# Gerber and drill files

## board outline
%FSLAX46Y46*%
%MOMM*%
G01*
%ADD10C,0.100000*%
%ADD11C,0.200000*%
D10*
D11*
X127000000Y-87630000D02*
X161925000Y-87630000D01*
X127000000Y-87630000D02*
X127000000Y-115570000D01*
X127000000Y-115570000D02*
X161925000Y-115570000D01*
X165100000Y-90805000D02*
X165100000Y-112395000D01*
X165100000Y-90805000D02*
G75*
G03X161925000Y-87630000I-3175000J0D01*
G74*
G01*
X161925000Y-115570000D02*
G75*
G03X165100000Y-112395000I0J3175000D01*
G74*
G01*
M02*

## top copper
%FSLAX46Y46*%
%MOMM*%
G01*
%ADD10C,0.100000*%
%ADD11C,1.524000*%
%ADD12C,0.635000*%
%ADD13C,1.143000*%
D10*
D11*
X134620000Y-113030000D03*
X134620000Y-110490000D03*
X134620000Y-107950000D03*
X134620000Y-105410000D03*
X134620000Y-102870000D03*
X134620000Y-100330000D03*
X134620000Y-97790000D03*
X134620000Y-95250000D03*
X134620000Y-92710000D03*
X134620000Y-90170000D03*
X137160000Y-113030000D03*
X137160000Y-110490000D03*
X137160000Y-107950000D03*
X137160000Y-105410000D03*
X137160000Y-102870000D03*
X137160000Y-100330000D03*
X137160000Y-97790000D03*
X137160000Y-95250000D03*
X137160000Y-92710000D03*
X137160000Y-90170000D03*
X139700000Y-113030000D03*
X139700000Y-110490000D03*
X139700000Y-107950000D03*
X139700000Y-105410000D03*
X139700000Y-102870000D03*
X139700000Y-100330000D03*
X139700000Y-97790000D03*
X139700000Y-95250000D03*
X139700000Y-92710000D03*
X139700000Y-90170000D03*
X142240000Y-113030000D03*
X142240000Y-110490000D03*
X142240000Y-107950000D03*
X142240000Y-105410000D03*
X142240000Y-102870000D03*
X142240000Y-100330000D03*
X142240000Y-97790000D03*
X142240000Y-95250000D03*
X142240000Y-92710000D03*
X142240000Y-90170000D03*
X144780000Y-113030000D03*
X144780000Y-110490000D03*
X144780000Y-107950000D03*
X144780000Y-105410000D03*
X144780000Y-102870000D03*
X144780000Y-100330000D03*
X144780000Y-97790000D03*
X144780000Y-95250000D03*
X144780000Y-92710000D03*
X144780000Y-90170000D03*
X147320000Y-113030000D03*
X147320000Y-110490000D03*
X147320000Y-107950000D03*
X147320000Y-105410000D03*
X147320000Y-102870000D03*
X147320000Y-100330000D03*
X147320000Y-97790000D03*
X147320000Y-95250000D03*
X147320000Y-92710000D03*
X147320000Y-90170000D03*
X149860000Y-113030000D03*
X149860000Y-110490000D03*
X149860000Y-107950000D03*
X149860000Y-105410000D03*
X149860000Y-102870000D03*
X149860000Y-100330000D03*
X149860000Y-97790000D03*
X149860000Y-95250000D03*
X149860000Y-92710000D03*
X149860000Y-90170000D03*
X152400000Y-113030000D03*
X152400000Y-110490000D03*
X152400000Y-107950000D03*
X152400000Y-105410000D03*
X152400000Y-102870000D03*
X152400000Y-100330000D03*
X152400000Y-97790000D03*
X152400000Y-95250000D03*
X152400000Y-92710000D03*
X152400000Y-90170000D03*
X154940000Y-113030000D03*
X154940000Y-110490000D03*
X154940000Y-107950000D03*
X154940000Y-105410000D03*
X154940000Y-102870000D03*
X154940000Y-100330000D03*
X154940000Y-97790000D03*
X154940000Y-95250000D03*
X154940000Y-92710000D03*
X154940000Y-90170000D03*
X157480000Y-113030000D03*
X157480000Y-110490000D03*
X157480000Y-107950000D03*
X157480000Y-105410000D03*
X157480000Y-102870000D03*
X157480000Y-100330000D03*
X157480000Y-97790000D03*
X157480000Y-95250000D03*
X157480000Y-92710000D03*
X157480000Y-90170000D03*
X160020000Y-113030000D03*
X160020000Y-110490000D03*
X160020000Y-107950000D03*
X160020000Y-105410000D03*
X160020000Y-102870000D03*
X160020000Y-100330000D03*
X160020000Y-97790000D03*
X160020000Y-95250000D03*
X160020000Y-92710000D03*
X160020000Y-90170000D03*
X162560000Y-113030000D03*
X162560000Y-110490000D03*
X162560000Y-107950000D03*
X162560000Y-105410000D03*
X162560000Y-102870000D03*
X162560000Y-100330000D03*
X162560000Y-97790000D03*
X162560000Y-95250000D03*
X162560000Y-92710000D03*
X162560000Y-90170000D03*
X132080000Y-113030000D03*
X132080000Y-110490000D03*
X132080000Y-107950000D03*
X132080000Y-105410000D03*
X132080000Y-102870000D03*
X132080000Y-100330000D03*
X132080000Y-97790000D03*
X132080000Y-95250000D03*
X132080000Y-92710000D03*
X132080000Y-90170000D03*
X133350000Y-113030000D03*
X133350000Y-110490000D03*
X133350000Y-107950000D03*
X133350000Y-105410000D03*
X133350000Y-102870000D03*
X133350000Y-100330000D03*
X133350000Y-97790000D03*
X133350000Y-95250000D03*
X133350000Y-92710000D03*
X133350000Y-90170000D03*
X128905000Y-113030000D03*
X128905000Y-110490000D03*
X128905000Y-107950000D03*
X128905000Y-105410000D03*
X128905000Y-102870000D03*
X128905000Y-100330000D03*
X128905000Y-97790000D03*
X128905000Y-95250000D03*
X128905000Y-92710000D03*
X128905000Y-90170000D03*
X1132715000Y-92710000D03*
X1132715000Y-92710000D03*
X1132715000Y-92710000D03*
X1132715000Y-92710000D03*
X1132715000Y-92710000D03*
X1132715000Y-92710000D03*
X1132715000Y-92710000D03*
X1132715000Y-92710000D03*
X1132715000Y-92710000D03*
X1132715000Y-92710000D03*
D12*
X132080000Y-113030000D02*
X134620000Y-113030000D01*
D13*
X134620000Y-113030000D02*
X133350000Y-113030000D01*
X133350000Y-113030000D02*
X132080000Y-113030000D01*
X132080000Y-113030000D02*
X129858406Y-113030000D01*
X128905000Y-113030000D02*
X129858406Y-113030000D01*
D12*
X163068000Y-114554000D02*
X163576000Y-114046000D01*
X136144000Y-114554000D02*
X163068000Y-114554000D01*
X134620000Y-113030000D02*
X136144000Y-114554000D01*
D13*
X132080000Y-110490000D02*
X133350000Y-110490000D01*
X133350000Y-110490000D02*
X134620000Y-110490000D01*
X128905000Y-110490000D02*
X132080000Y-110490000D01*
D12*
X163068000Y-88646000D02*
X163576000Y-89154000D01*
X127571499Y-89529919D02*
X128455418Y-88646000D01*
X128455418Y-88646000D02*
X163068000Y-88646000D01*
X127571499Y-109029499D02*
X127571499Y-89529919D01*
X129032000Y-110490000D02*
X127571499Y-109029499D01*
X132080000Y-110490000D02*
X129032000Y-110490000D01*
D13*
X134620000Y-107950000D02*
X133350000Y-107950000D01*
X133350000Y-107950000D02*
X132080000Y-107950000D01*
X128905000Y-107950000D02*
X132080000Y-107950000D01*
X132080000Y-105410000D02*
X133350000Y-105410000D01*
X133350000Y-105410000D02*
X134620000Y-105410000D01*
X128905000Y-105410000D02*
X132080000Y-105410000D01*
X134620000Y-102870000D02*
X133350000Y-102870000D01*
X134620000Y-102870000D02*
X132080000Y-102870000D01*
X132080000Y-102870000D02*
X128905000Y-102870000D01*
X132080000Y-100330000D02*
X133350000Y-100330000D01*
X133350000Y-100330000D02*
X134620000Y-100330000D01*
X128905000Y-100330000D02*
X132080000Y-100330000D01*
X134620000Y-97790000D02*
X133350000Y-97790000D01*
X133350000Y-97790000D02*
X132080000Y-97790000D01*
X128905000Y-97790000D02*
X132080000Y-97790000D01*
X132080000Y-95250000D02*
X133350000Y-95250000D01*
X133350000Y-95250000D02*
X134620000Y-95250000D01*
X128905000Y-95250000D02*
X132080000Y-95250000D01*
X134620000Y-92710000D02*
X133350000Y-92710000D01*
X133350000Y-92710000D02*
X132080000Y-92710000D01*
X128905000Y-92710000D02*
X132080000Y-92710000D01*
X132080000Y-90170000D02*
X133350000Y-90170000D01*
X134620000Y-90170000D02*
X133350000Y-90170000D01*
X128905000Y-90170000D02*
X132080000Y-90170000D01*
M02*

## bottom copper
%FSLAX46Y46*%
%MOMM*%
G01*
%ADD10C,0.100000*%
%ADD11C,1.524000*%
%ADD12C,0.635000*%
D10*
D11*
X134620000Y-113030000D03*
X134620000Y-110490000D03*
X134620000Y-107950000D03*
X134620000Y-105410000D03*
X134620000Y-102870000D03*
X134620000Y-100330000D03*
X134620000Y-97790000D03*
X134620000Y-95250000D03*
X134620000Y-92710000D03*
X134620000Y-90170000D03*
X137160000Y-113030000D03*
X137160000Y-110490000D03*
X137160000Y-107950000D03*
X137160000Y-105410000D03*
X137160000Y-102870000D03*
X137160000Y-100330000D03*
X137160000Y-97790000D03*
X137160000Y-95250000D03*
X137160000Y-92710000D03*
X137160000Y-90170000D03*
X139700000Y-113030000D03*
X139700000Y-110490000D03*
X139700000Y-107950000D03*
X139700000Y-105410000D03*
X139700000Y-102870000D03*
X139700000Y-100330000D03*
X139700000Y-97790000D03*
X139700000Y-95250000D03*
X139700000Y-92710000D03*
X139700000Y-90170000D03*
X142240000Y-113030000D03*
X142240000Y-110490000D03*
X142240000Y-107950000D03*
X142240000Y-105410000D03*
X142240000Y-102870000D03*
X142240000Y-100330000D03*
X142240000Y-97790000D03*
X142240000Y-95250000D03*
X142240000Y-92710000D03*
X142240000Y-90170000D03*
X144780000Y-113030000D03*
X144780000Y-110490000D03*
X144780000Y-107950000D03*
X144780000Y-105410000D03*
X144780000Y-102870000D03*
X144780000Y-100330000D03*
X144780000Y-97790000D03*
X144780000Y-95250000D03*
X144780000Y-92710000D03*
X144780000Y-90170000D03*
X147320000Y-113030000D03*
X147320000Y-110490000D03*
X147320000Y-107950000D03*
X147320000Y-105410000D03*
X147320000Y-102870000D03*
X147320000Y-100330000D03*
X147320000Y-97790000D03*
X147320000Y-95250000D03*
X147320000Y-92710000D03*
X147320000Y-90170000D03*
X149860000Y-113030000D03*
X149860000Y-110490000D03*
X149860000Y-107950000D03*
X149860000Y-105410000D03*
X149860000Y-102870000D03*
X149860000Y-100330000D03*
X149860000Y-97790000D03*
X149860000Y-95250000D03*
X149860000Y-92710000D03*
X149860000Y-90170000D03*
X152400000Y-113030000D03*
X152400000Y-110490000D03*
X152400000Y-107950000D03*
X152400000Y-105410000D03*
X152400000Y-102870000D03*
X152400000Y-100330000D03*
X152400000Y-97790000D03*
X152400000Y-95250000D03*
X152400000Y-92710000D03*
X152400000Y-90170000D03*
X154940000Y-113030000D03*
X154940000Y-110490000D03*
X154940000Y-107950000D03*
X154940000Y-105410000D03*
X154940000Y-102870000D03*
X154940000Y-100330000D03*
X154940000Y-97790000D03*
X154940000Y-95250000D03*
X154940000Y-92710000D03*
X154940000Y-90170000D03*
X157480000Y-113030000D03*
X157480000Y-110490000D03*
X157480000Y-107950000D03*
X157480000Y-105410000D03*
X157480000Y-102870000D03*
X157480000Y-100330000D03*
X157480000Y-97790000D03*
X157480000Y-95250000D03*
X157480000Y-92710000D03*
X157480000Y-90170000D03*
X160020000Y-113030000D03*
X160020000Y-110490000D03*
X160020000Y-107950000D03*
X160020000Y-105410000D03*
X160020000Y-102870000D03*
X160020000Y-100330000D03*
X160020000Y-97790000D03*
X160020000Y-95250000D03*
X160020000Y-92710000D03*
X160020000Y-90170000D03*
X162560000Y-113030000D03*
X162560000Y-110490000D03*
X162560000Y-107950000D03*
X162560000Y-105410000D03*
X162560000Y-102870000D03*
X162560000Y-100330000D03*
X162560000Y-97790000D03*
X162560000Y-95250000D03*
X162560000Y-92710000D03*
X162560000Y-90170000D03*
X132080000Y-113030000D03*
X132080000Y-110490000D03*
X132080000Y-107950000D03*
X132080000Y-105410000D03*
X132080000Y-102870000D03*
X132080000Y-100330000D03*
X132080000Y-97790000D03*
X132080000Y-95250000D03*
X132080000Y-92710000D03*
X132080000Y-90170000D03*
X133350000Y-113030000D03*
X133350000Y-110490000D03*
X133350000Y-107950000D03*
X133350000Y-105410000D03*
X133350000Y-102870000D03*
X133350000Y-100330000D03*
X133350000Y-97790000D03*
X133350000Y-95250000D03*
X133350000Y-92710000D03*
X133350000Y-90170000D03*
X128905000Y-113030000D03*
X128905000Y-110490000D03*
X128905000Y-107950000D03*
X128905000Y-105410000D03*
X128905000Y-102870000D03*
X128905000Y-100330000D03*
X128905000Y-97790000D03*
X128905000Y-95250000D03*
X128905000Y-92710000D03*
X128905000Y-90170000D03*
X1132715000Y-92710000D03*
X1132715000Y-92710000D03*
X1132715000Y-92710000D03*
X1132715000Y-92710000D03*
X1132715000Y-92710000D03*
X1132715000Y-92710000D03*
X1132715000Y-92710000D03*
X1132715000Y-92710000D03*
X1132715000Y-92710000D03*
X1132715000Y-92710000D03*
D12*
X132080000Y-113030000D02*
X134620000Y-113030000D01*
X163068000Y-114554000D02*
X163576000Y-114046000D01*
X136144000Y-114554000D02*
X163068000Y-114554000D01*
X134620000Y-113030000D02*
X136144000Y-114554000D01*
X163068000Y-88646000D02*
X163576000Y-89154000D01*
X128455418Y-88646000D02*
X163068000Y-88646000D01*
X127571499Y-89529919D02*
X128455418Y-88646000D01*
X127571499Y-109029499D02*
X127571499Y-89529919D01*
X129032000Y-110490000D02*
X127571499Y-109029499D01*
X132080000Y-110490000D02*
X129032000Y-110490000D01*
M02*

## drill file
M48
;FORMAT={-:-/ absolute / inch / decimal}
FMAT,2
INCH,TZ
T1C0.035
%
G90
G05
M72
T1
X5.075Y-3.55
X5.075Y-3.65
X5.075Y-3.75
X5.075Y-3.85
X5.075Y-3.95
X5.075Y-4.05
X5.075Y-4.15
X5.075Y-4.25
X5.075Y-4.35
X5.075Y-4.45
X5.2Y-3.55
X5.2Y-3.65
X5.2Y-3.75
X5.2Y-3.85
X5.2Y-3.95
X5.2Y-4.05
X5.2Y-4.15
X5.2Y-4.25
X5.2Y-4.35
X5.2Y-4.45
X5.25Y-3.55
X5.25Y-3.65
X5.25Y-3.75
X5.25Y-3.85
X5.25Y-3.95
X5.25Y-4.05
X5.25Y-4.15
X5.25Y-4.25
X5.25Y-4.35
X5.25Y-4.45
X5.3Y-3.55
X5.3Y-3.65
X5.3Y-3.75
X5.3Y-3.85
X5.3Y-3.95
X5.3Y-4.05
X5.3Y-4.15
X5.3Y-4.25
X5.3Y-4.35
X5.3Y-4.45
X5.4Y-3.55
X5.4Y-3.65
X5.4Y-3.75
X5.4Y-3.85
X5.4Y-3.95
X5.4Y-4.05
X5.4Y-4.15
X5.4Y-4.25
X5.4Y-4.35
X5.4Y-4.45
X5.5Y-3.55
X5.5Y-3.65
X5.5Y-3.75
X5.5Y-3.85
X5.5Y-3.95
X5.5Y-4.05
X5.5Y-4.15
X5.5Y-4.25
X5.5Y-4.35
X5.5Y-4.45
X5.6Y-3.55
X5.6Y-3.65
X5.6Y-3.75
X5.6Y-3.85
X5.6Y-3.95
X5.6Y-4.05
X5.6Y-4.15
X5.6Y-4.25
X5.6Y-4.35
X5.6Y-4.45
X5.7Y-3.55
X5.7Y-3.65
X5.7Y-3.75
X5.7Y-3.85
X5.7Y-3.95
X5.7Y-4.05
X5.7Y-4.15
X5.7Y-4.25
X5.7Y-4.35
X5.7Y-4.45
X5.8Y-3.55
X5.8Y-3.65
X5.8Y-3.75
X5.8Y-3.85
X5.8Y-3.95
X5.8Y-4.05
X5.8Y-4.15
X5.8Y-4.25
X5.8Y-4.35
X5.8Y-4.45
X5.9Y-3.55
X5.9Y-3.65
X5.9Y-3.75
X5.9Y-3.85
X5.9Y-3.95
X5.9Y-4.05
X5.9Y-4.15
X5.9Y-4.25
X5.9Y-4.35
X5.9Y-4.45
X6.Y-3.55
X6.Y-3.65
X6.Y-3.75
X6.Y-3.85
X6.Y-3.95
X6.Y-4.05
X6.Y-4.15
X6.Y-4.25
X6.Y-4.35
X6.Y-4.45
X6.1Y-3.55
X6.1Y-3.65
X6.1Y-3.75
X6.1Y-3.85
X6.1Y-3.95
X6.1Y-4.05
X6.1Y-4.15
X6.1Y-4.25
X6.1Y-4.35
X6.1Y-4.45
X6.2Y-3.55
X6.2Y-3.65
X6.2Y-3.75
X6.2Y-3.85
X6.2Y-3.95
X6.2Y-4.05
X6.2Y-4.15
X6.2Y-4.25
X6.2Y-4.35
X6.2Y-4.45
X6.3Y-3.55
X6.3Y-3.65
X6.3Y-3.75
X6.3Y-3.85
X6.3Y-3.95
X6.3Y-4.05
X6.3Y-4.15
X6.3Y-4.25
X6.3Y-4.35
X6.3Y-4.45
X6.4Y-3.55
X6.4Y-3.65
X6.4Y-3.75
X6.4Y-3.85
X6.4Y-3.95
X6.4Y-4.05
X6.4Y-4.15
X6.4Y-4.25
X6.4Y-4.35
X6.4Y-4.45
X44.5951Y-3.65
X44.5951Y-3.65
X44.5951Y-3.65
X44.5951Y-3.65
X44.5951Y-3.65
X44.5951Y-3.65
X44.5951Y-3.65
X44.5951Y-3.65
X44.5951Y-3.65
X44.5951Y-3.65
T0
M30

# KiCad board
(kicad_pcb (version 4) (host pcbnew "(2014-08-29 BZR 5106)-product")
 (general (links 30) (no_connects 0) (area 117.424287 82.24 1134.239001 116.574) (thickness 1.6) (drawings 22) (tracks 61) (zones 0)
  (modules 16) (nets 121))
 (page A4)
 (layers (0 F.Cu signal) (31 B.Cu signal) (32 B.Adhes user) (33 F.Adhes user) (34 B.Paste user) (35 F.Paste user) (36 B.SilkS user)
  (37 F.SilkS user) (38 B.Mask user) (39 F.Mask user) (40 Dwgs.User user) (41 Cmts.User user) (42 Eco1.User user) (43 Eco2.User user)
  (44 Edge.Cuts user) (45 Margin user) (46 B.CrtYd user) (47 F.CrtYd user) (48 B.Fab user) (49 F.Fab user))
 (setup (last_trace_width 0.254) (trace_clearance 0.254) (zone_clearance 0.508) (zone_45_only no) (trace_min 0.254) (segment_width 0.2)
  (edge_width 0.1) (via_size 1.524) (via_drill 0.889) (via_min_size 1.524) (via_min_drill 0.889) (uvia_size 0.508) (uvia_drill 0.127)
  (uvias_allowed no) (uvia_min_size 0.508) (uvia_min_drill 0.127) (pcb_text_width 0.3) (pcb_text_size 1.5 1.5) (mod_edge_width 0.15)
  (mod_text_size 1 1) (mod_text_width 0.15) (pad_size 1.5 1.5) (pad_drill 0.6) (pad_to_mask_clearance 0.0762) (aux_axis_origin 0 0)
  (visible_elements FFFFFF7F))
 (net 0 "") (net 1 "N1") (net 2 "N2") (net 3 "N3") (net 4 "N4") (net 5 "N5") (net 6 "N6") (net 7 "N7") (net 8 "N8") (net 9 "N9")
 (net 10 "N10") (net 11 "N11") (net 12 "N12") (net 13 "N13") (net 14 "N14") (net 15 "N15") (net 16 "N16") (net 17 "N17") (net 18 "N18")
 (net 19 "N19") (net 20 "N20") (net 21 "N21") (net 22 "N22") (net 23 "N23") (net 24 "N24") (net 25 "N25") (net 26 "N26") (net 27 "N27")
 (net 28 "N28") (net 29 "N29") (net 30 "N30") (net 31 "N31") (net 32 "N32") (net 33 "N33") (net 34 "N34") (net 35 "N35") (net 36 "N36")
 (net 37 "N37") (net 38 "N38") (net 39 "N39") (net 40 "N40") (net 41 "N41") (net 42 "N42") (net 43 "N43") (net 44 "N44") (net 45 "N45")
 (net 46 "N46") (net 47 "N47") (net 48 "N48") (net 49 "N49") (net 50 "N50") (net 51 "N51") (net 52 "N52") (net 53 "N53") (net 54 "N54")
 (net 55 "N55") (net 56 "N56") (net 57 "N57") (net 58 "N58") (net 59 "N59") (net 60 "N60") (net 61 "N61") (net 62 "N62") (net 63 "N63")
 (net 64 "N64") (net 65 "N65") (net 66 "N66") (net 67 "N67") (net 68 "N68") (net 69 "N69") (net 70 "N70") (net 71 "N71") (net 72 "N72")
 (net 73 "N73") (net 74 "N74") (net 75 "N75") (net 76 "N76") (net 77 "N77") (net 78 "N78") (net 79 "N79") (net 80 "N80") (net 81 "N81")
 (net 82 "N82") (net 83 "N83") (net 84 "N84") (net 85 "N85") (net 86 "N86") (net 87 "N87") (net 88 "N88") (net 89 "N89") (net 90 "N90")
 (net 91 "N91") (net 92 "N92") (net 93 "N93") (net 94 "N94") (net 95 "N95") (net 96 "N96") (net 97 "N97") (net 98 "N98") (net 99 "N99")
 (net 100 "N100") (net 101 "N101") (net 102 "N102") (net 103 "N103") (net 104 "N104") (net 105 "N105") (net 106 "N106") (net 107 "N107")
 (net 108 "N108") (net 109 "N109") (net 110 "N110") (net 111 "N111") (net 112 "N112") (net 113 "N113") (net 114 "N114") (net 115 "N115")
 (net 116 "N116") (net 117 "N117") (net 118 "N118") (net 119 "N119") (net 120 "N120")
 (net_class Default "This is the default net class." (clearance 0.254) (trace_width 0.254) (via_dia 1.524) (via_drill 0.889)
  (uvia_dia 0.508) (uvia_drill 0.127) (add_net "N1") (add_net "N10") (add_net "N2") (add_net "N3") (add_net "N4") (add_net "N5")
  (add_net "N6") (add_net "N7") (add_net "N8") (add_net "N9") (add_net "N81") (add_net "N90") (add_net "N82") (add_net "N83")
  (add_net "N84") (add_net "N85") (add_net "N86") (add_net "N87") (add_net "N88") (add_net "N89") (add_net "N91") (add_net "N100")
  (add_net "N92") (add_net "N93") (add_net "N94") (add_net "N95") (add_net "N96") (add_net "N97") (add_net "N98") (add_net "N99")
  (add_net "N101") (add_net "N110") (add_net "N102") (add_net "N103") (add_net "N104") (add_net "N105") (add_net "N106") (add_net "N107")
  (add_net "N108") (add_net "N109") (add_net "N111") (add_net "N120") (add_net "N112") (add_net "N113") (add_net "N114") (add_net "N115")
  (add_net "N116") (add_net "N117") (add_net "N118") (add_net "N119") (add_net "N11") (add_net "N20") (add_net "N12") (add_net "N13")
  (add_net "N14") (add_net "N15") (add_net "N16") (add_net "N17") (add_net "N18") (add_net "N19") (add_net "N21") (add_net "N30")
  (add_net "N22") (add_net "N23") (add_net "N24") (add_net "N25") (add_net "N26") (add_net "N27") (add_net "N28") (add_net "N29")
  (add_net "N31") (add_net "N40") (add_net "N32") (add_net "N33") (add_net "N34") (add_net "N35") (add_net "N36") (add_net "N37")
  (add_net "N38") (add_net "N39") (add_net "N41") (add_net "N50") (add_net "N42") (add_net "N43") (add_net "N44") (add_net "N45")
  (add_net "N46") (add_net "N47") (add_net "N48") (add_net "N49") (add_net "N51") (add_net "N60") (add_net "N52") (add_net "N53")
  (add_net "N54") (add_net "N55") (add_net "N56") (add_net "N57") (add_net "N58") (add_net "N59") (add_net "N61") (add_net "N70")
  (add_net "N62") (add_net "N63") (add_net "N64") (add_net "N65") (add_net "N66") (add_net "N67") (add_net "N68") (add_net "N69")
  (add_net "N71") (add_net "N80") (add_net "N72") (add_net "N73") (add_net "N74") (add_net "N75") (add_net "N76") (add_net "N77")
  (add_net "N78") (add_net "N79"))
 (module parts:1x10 (layer F.Cu) (at 134.62 101.6 90)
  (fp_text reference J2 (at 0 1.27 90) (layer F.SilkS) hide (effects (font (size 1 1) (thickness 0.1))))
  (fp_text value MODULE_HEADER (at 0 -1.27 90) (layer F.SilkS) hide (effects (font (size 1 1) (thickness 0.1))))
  (pad 1 thru_hole circle (at -11.43 0 90) (size 1.524 1.524) (drill 0.889) (layers *.Cu *.Mask F.SilkS) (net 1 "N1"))
  (pad 2 thru_hole circle (at -8.89 0 90) (size 1.524 1.524) (drill 0.889) (layers *.Cu *.Mask F.SilkS) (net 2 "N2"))
  (pad 3 thru_hole circle (at -6.35 0 90) (size 1.524 1.524) (drill 0.889) (layers *.Cu *.Mask F.SilkS) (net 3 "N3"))
  (pad 4 thru_hole circle (at -3.81 0 90) (size 1.524 1.524) (drill 0.889) (layers *.Cu *.Mask F.SilkS) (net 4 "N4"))
  (pad 5 thru_hole circle (at -1.27 0 90) (size 1.524 1.524) (drill 0.889) (layers *.Cu *.Mask F.SilkS) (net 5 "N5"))
  (pad 6 thru_hole circle (at 1.27 0 90) (size 1.524 1.524) (drill 0.889) (layers *.Cu *.Mask F.SilkS) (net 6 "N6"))
  (pad 7 thru_hole circle (at 3.81 0 90) (size 1.524 1.524) (drill 0.889) (layers *.Cu *.Mask F.SilkS) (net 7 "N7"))
  (pad 8 thru_hole circle (at 6.35 0 90) (size 1.524 1.524) (drill 0.889) (layers *.Cu *.Mask F.SilkS) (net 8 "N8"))
  (pad 9 thru_hole circle (at 8.89 0 90) (size 1.524 1.524) (drill 0.889) (layers *.Cu *.Mask F.SilkS) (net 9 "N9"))
  (pad 10 thru_hole circle (at 11.43 0 90) (size 1.524 1.524) (drill 0.889) (layers *.Cu *.Mask F.SilkS) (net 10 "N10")))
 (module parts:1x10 (layer F.Cu) (at 137.16 101.6 90)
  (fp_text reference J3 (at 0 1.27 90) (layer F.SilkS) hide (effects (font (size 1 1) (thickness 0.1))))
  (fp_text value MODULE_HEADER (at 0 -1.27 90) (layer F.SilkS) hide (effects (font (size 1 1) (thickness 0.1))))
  (pad 1 thru_hole circle (at -11.43 0 90) (size 1.524 1.524) (drill 0.889) (layers *.Cu *.Mask F.SilkS) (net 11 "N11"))
  (pad 2 thru_hole circle (at -8.89 0 90) (size 1.524 1.524) (drill 0.889) (layers *.Cu *.Mask F.SilkS) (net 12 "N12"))
  (pad 3 thru_hole circle (at -6.35 0 90) (size 1.524 1.524) (drill 0.889) (layers *.Cu *.Mask F.SilkS) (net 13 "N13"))
  (pad 4 thru_hole circle (at -3.81 0 90) (size 1.524 1.524) (drill 0.889) (layers *.Cu *.Mask F.SilkS) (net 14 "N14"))
  (pad 5 thru_hole circle (at -1.27 0 90) (size 1.524 1.524) (drill 0.889) (layers *.Cu *.Mask F.SilkS) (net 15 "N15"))
  (pad 6 thru_hole circle (at 1.27 0 90) (size 1.524 1.524) (drill 0.889) (layers *.Cu *.Mask F.SilkS) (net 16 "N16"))
  (pad 7 thru_hole circle (at 3.81 0 90) (size 1.524 1.524) (drill 0.889) (layers *.Cu *.Mask F.SilkS) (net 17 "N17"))
  (pad 8 thru_hole circle (at 6.35 0 90) (size 1.524 1.524) (drill 0.889) (layers *.Cu *.Mask F.SilkS) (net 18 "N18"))
  (pad 9 thru_hole circle (at 8.89 0 90) (size 1.524 1.524) (drill 0.889) (layers *.Cu *.Mask F.SilkS) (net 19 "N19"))
  (pad 10 thru_hole circle (at 11.43 0 90) (size 1.524 1.524) (drill 0.889) (layers *.Cu *.Mask F.SilkS) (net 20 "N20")))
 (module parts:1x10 (layer F.Cu) (at 139.7 101.6 90)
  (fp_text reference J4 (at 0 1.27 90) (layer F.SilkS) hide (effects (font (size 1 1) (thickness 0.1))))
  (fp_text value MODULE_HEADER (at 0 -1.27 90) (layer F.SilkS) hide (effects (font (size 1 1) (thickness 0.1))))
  (pad 1 thru_hole circle (at -11.43 0 90) (size 1.524 1.524) (drill 0.889) (layers *.Cu *.Mask F.SilkS) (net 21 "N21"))
  (pad 2 thru_hole circle (at -8.89 0 90) (size 1.524 1.524) (drill 0.889) (layers *.Cu *.Mask F.SilkS) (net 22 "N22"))
  (pad 3 thru_hole circle (at -6.35 0 90) (size 1.524 1.524) (drill 0.889) (layers *.Cu *.Mask F.SilkS) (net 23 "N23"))
  (pad 4 thru_hole circle (at -3.81 0 90) (size 1.524 1.524) (drill 0.889) (layers *.Cu *.Mask F.SilkS) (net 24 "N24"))
  (pad 5 thru_hole circle (at -1.27 0 90) (size 1.524 1.524) (drill 0.889) (layers *.Cu *.Mask F.SilkS) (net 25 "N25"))
  (pad 6 thru_hole circle (at 1.27 0 90) (size 1.524 1.524) (drill 0.889) (layers *.Cu *.Mask F.SilkS) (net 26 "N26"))
  (pad 7 thru_hole circle (at 3.81 0 90) (size 1.524 1.524) (drill 0.889) (layers *.Cu *.Mask F.SilkS) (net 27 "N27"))
  (pad 8 thru_hole circle (at 6.35 0 90) (size 1.524 1.524) (drill 0.889) (layers *.Cu *.Mask F.SilkS) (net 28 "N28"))
  (pad 9 thru_hole circle (at 8.89 0 90) (size 1.524 1.524) (drill 0.889) (layers *.Cu *.Mask F.SilkS) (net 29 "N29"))
  (pad 10 thru_hole circle (at 11.43 0 90) (size 1.524 1.524) (drill 0.889) (layers *.Cu *.Mask F.SilkS) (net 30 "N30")))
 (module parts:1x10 (layer F.Cu) (at 142.24 101.6 90)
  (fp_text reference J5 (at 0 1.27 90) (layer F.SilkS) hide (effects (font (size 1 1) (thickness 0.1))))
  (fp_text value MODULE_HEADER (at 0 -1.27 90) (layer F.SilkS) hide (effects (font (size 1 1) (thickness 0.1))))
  (pad 1 thru_hole circle (at -11.43 0 90) (size 1.524 1.524) (drill 0.889) (layers *.Cu *.Mask F.SilkS) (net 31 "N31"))
  (pad 2 thru_hole circle (at -8.89 0 90) (size 1.524 1.524) (drill 0.889) (layers *.Cu *.Mask F.SilkS) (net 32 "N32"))
  (pad 3 thru_hole circle (at -6.35 0 90) (size 1.524 1.524) (drill 0.889) (layers *.Cu *.Mask F.SilkS) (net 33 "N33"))
  (pad 4 thru_hole circle (at -3.81 0 90) (size 1.524 1.524) (drill 0.889) (layers *.Cu *.Mask F.SilkS) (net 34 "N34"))
  (pad 5 thru_hole circle (at -1.27 0 90) (size 1.524 1.524) (drill 0.889) (layers *.Cu *.Mask F.SilkS) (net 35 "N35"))
  (pad 6 thru_hole circle (at 1.27 0 90) (size 1.524 1.524) (drill 0.889) (layers *.Cu *.Mask F.SilkS) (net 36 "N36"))
  (pad 7 thru_hole circle (at 3.81 0 90) (size 1.524 1.524) (drill 0.889) (layers *.Cu *.Mask F.SilkS) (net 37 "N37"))
  (pad 8 thru_hole circle (at 6.35 0 90) (size 1.524 1.524) (drill 0.889) (layers *.Cu *.Mask F.SilkS) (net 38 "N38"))
  (pad 9 thru_hole circle (at 8.89 0 90) (size 1.524 1.524) (drill 0.889) (layers *.Cu *.Mask F.SilkS) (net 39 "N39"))
  (pad 10 thru_hole circle (at 11.43 0 90) (size 1.524 1.524) (drill 0.889) (layers *.Cu *.Mask F.SilkS) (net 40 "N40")))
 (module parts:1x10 (layer F.Cu) (at 144.78 101.6 90)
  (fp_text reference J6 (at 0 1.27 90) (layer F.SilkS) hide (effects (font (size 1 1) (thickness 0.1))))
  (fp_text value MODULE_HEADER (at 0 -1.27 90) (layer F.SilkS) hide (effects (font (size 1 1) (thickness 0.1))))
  (pad 1 thru_hole circle (at -11.43 0 90) (size 1.524 1.524) (drill 0.889) (layers *.Cu *.Mask F.SilkS) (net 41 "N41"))
  (pad 2 thru_hole circle (at -8.89 0 90) (size 1.524 1.524) (drill 0.889) (layers *.Cu *.Mask F.SilkS) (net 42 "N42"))
  (pad 3 thru_hole circle (at -6.35 0 90) (size 1.524 1.524) (drill 0.889) (layers *.Cu *.Mask F.SilkS) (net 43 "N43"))
  (pad 4 thru_hole circle (at -3.81 0 90) (size 1.524 1.524) (drill 0.889) (layers *.Cu *.Mask F.SilkS) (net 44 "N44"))
  (pad 5 thru_hole circle (at -1.27 0 90) (size 1.524 1.524) (drill 0.889) (layers *.Cu *.Mask F.SilkS) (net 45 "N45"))
  (pad 6 thru_hole circle (at 1.27 0 90) (size 1.524 1.524) (drill 0.889) (layers *.Cu *.Mask F.SilkS) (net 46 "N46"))
  (pad 7 thru_hole circle (at 3.81 0 90) (size 1.524 1.524) (drill 0.889) (layers *.Cu *.Mask F.SilkS) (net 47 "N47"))
  (pad 8 thru_hole circle (at 6.35 0 90) (size 1.524 1.524) (drill 0.889) (layers *.Cu *.Mask F.SilkS) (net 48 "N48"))
  (pad 9 thru_hole circle (at 8.89 0 90) (size 1.524 1.524) (drill 0.889) (layers *.Cu *.Mask F.SilkS) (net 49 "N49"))
  (pad 10 thru_hole circle (at 11.43 0 90) (size 1.524 1.524) (drill 0.889) (layers *.Cu *.Mask F.SilkS) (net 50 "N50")))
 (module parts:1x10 (layer F.Cu) (at 147.32 101.6 90)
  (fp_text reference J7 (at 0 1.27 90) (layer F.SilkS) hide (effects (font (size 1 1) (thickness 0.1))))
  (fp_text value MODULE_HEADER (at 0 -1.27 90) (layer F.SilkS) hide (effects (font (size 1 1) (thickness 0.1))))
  (pad 1 thru_hole circle (at -11.43 0 90) (size 1.524 1.524) (drill 0.889) (layers *.Cu *.Mask F.SilkS) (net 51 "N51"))
  (pad 2 thru_hole circle (at -8.89 0 90) (size 1.524 1.524) (drill 0.889) (layers *.Cu *.Mask F.SilkS) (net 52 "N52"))
  (pad 3 thru_hole circle (at -6.35 0 90) (size 1.524 1.524) (drill 0.889) (layers *.Cu *.Mask F.SilkS) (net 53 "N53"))
  (pad 4 thru_hole circle (at -3.81 0 90) (size 1.524 1.524) (drill 0.889) (layers *.Cu *.Mask F.SilkS) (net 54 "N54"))
  (pad 5 thru_hole circle (at -1.27 0 90) (size 1.524 1.524) (drill 0.889) (layers *.Cu *.Mask F.SilkS) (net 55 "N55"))
  (pad 6 thru_hole circle (at 1.27 0 90) (size 1.524 1.524) (drill 0.889) (layers *.Cu *.Mask F.SilkS) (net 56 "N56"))
  (pad 7 thru_hole circle (at 3.81 0 90) (size 1.524 1.524) (drill 0.889) (layers *.Cu *.Mask F.SilkS) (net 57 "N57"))
  (pad 8 thru_hole circle (at 6.35 0 90) (size 1.524 1.524) (drill 0.889) (layers *.Cu *.Mask F.SilkS) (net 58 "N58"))
  (pad 9 thru_hole circle (at 8.89 0 90) (size 1.524 1.524) (drill 0.889) (layers *.Cu *.Mask F.SilkS) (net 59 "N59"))
  (pad 10 thru_hole circle (at 11.43 0 90) (size 1.524 1.524) (drill 0.889) (layers *.Cu *.Mask F.SilkS) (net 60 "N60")))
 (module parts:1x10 (layer F.Cu) (at 149.86 101.6 90)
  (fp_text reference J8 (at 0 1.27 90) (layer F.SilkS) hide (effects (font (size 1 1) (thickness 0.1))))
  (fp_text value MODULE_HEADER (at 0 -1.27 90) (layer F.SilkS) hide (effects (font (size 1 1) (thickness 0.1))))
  (pad 1 thru_hole circle (at -11.43 0 90) (size 1.524 1.524) (drill 0.889) (layers *.Cu *.Mask F.SilkS) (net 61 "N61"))
  (pad 2 thru_hole circle (at -8.89 0 90) (size 1.524 1.524) (drill 0.889) (layers *.Cu *.Mask F.SilkS) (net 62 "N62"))
  (pad 3 thru_hole circle (at -6.35 0 90) (size 1.524 1.524) (drill 0.889) (layers *.Cu *.Mask F.SilkS) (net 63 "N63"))
  (pad 4 thru_hole circle (at -3.81 0 90) (size 1.524 1.524) (drill 0.889) (layers *.Cu *.Mask F.SilkS) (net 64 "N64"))
  (pad 5 thru_hole circle (at -1.27 0 90) (size 1.524 1.524) (drill 0.889) (layers *.Cu *.Mask F.SilkS) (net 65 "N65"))
  (pad 6 thru_hole circle (at 1.27 0 90) (size 1.524 1.524) (drill 0.889) (layers *.Cu *.Mask F.SilkS) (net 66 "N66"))
  (pad 7 thru_hole circle (at 3.81 0 90) (size 1.524 1.524) (drill 0.889) (layers *.Cu *.Mask F.SilkS) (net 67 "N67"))
  (pad 8 thru_hole circle (at 6.35 0 90) (size 1.524 1.524) (drill 0.889) (layers *.Cu *.Mask F.SilkS) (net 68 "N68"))
  (pad 9 thru_hole circle (at 8.89 0 90) (size 1.524 1.524) (drill 0.889) (layers *.Cu *.Mask F.SilkS) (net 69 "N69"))
  (pad 10 thru_hole circle (at 11.43 0 90) (size 1.524 1.524) (drill 0.889) (layers *.Cu *.Mask F.SilkS) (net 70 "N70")))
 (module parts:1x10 (layer F.Cu) (at 152.4 101.6 90)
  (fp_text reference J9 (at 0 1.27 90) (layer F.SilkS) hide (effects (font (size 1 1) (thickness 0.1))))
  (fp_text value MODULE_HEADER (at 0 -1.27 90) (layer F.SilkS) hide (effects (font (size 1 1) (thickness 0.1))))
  (pad 1 thru_hole circle (at -11.43 0 90) (size 1.524 1.524) (drill 0.889) (layers *.Cu *.Mask F.SilkS) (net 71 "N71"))
  (pad 2 thru_hole circle (at -8.89 0 90) (size 1.524 1.524) (drill 0.889) (layers *.Cu *.Mask F.SilkS) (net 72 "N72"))
  (pad 3 thru_hole circle (at -6.35 0 90) (size 1.524 1.524) (drill 0.889) (layers *.Cu *.Mask F.SilkS) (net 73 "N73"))
  (pad 4 thru_hole circle (at -3.81 0 90) (size 1.524 1.524) (drill 0.889) (layers *.Cu *.Mask F.SilkS) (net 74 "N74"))
  (pad 5 thru_hole circle (at -1.27 0 90) (size 1.524 1.524) (drill 0.889) (layers *.Cu *.Mask F.SilkS) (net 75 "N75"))
  (pad 6 thru_hole circle (at 1.27 0 90) (size 1.524 1.524) (drill 0.889) (layers *.Cu *.Mask F.SilkS) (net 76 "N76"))
  (pad 7 thru_hole circle (at 3.81 0 90) (size 1.524 1.524) (drill 0.889) (layers *.Cu *.Mask F.SilkS) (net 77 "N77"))
  (pad 8 thru_hole circle (at 6.35 0 90) (size 1.524 1.524) (drill 0.889) (layers *.Cu *.Mask F.SilkS) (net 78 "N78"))
  (pad 9 thru_hole circle (at 8.89 0 90) (size 1.524 1.524) (drill 0.889) (layers *.Cu *.Mask F.SilkS) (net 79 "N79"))
  (pad 10 thru_hole circle (at 11.43 0 90) (size 1.524 1.524) (drill 0.889) (layers *.Cu *.Mask F.SilkS) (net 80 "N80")))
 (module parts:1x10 (layer F.Cu) (at 154.94 101.6 90)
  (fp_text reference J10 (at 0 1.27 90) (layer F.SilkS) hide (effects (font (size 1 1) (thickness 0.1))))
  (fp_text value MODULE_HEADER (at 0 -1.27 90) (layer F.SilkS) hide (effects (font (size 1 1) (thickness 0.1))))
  (pad 1 thru_hole circle (at -11.43 0 90) (size 1.524 1.524) (drill 0.889) (layers *.Cu *.Mask F.SilkS) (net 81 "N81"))
  (pad 2 thru_hole circle (at -8.89 0 90) (size 1.524 1.524) (drill 0.889) (layers *.Cu *.Mask F.SilkS) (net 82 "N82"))
  (pad 3 thru_hole circle (at -6.35 0 90) (size 1.524 1.524) (drill 0.889) (layers *.Cu *.Mask F.SilkS) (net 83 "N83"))
  (pad 4 thru_hole circle (at -3.81 0 90) (size 1.524 1.524) (drill 0.889) (layers *.Cu *.Mask F.SilkS) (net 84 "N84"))
  (pad 5 thru_hole circle (at -1.27 0 90) (size 1.524 1.524) (drill 0.889) (layers *.Cu *.Mask F.SilkS) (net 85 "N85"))
  (pad 6 thru_hole circle (at 1.27 0 90) (size 1.524 1.524) (drill 0.889) (layers *.Cu *.Mask F.SilkS) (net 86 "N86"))
  (pad 7 thru_hole circle (at 3.81 0 90) (size 1.524 1.524) (drill 0.889) (layers *.Cu *.Mask F.SilkS) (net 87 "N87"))
  (pad 8 thru_hole circle (at 6.35 0 90) (size 1.524 1.524) (drill 0.889) (layers *.Cu *.Mask F.SilkS) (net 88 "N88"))
  (pad 9 thru_hole circle (at 8.89 0 90) (size 1.524 1.524) (drill 0.889) (layers *.Cu *.Mask F.SilkS) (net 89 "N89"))
  (pad 10 thru_hole circle (at 11.43 0 90) (size 1.524 1.524) (drill 0.889) (layers *.Cu *.Mask F.SilkS) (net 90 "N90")))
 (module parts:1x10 (layer F.Cu) (at 157.48 101.6 90)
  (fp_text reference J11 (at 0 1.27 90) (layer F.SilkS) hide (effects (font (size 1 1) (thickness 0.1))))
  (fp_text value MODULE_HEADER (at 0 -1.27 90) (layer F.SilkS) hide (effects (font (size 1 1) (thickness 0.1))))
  (pad 1 thru_hole circle (at -11.43 0 90) (size 1.524 1.524) (drill 0.889) (layers *.Cu *.Mask F.SilkS) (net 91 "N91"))
  (pad 2 thru_hole circle (at -8.89 0 90) (size 1.524 1.524) (drill 0.889) (layers *.Cu *.Mask F.SilkS) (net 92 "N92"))
  (pad 3 thru_hole circle (at -6.35 0 90) (size 1.524 1.524) (drill 0.889) (layers *.Cu *.Mask F.SilkS) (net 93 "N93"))
  (pad 4 thru_hole circle (at -3.81 0 90) (size 1.524 1.524) (drill 0.889) (layers *.Cu *.Mask F.SilkS) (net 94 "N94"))
  (pad 5 thru_hole circle (at -1.27 0 90) (size 1.524 1.524) (drill 0.889) (layers *.Cu *.Mask F.SilkS) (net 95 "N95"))
  (pad 6 thru_hole circle (at 1.27 0 90) (size 1.524 1.524) (drill 0.889) (layers *.Cu *.Mask F.SilkS) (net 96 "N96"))
  (pad 7 thru_hole circle (at 3.81 0 90) (size 1.524 1.524) (drill 0.889) (layers *.Cu *.Mask F.SilkS) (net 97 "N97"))
  (pad 8 thru_hole circle (at 6.35 0 90) (size 1.524 1.524) (drill 0.889) (layers *.Cu *.Mask F.SilkS) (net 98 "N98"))
  (pad 9 thru_hole circle (at 8.89 0 90) (size 1.524 1.524) (drill 0.889) (layers *.Cu *.Mask F.SilkS) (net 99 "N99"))
  (pad 10 thru_hole circle (at 11.43 0 90) (size 1.524 1.524) (drill 0.889) (layers *.Cu *.Mask F.SilkS) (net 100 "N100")))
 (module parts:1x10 (layer F.Cu) (at 160.02 101.6 90)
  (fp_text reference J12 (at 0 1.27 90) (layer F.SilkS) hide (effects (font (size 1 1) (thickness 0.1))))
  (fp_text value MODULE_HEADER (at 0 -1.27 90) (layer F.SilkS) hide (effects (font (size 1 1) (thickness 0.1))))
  (pad 1 thru_hole circle (at -11.43 0 90) (size 1.524 1.524) (drill 0.889) (layers *.Cu *.Mask F.SilkS) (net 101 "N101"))
  (pad 2 thru_hole circle (at -8.89 0 90) (size 1.524 1.524) (drill 0.889) (layers *.Cu *.Mask F.SilkS) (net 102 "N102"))
  (pad 3 thru_hole circle (at -6.35 0 90) (size 1.524 1.524) (drill 0.889) (layers *.Cu *.Mask F.SilkS) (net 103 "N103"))
  (pad 4 thru_hole circle (at -3.81 0 90) (size 1.524 1.524) (drill 0.889) (layers *.Cu *.Mask F.SilkS) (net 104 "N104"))
  (pad 5 thru_hole circle (at -1.27 0 90) (size 1.524 1.524) (drill 0.889) (layers *.Cu *.Mask F.SilkS) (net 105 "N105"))
  (pad 6 thru_hole circle (at 1.27 0 90) (size 1.524 1.524) (drill 0.889) (layers *.Cu *.Mask F.SilkS) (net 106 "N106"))
  (pad 7 thru_hole circle (at 3.81 0 90) (size 1.524 1.524) (drill 0.889) (layers *.Cu *.Mask F.SilkS) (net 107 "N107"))
  (pad 8 thru_hole circle (at 6.35 0 90) (size 1.524 1.524) (drill 0.889) (layers *.Cu *.Mask F.SilkS) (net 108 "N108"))
  (pad 9 thru_hole circle (at 8.89 0 90) (size 1.524 1.524) (drill 0.889) (layers *.Cu *.Mask F.SilkS) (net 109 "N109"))
  (pad 10 thru_hole circle (at 11.43 0 90) (size 1.524 1.524) (drill 0.889) (layers *.Cu *.Mask F.SilkS) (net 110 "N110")))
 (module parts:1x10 (layer F.Cu) (at 162.56 101.6 90)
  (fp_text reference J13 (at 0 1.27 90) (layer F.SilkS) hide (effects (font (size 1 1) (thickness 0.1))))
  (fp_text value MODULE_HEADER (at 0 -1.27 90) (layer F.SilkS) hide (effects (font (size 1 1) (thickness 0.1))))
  (pad 1 thru_hole circle (at -11.43 0 90) (size 1.524 1.524) (drill 0.889) (layers *.Cu *.Mask F.SilkS) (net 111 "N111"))
  (pad 2 thru_hole circle (at -8.89 0 90) (size 1.524 1.524) (drill 0.889) (layers *.Cu *.Mask F.SilkS) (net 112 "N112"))
  (pad 3 thru_hole circle (at -6.35 0 90) (size 1.524 1.524) (drill 0.889) (layers *.Cu *.Mask F.SilkS) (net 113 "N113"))
  (pad 4 thru_hole circle (at -3.81 0 90) (size 1.524 1.524) (drill 0.889) (layers *.Cu *.Mask F.SilkS) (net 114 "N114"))
  (pad 5 thru_hole circle (at -1.27 0 90) (size 1.524 1.524) (drill 0.889) (layers *.Cu *.Mask F.SilkS) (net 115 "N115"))
  (pad 6 thru_hole circle (at 1.27 0 90) (size 1.524 1.524) (drill 0.889) (layers *.Cu *.Mask F.SilkS) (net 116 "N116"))
  (pad 7 thru_hole circle (at 3.81 0 90) (size 1.524 1.524) (drill 0.889) (layers *.Cu *.Mask F.SilkS) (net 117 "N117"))
  (pad 8 thru_hole circle (at 6.35 0 90) (size 1.524 1.524) (drill 0.889) (layers *.Cu *.Mask F.SilkS) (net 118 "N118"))
  (pad 9 thru_hole circle (at 8.89 0 90) (size 1.524 1.524) (drill 0.889) (layers *.Cu *.Mask F.SilkS) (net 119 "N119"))
  (pad 10 thru_hole circle (at 11.43 0 90) (size 1.524 1.524) (drill 0.889) (layers *.Cu *.Mask F.SilkS) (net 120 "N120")))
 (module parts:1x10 (layer F.Cu) (at 132.08 101.6 90)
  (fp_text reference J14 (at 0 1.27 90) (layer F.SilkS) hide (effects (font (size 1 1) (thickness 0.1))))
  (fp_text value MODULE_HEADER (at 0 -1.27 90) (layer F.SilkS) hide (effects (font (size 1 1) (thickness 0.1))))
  (pad 1 thru_hole circle (at -11.43 0 90) (size 1.524 1.524) (drill 0.889) (layers *.Cu *.Mask F.SilkS) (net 1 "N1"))
  (pad 2 thru_hole circle (at -8.89 0 90) (size 1.524 1.524) (drill 0.889) (layers *.Cu *.Mask F.SilkS) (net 2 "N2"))
  (pad 3 thru_hole circle (at -6.35 0 90) (size 1.524 1.524) (drill 0.889) (layers *.Cu *.Mask F.SilkS) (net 3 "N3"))
  (pad 4 thru_hole circle (at -3.81 0 90) (size 1.524 1.524) (drill 0.889) (layers *.Cu *.Mask F.SilkS) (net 4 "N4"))
  (pad 5 thru_hole circle (at -1.27 0 90) (size 1.524 1.524) (drill 0.889) (layers *.Cu *.Mask F.SilkS) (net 5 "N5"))
  (pad 6 thru_hole circle (at 1.27 0 90) (size 1.524 1.524) (drill 0.889) (layers *.Cu *.Mask F.SilkS) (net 6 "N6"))
  (pad 7 thru_hole circle (at 3.81 0 90) (size 1.524 1.524) (drill 0.889) (layers *.Cu *.Mask F.SilkS) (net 7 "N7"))
  (pad 8 thru_hole circle (at 6.35 0 90) (size 1.524 1.524) (drill 0.889) (layers *.Cu *.Mask F.SilkS) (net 8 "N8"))
  (pad 9 thru_hole circle (at 8.89 0 90) (size 1.524 1.524) (drill 0.889) (layers *.Cu *.Mask F.SilkS) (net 9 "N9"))
  (pad 10 thru_hole circle (at 11.43 0 90) (size 1.524 1.524) (drill 0.889) (layers *.Cu *.Mask F.SilkS) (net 10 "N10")))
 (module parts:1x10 (layer F.Cu) (at 133.35 101.6 90)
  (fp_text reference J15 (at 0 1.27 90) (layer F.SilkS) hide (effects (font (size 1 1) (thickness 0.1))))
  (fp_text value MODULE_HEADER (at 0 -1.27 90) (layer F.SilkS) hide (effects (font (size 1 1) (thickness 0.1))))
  (pad 1 thru_hole circle (at -11.43 0 90) (size 1.524 1.524) (drill 0.889) (layers *.Cu *.Mask F.SilkS) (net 1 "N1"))
  (pad 2 thru_hole circle (at -8.89 0 90) (size 1.524 1.524) (drill 0.889) (layers *.Cu *.Mask F.SilkS) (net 2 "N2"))
  (pad 3 thru_hole circle (at -6.35 0 90) (size 1.524 1.524) (drill 0.889) (layers *.Cu *.Mask F.SilkS) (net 3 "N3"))
  (pad 4 thru_hole circle (at -3.81 0 90) (size 1.524 1.524) (drill 0.889) (layers *.Cu *.Mask F.SilkS) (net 4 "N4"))
  (pad 5 thru_hole circle (at -1.27 0 90) (size 1.524 1.524) (drill 0.889) (layers *.Cu *.Mask F.SilkS) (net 5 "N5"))
  (pad 6 thru_hole circle (at 1.27 0 90) (size 1.524 1.524) (drill 0.889) (layers *.Cu *.Mask F.SilkS) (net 6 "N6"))
  (pad 7 thru_hole circle (at 3.81 0 90) (size 1.524 1.524) (drill 0.889) (layers *.Cu *.Mask F.SilkS) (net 7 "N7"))
  (pad 8 thru_hole circle (at 6.35 0 90) (size 1.524 1.524) (drill 0.889) (layers *.Cu *.Mask F.SilkS) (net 8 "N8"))
  (pad 9 thru_hole circle (at 8.89 0 90) (size 1.524 1.524) (drill 0.889) (layers *.Cu *.Mask F.SilkS) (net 9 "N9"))
  (pad 10 thru_hole circle (at 11.43 0 90) (size 1.524 1.524) (drill 0.889) (layers *.Cu *.Mask F.SilkS) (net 10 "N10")))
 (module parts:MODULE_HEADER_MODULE (layer F.Cu) (at 128.905 101.6 90)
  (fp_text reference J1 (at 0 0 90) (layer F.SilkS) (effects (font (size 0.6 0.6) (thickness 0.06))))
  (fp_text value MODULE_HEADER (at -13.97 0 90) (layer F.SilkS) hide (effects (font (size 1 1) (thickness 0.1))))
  (pad 1 thru_hole circle (at -11.43 0 90) (size 1.524 1.524) (drill 0.889) (layers *.Cu *.Mask F.SilkS) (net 1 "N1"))
  (pad 2 thru_hole circle (at -8.89 0 90) (size 1.524 1.524) (drill 0.889) (layers *.Cu *.Mask F.SilkS) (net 2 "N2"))
  (pad 3 thru_hole circle (at -6.35 0 90) (size 1.524 1.524) (drill 0.889) (layers *.Cu *.Mask F.SilkS) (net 3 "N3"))
  (pad 4 thru_hole circle (at -3.81 0 90) (size 1.524 1.524) (drill 0.889) (layers *.Cu *.Mask F.SilkS) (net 4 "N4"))
  (pad 5 thru_hole circle (at -1.27 0 90) (size 1.524 1.524) (drill 0.889) (layers *.Cu *.Mask F.SilkS) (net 5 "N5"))
  (pad 6 thru_hole circle (at 1.27 0 90) (size 1.524 1.524) (drill 0.889) (layers *.Cu *.Mask F.SilkS) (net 6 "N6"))
  (pad 7 thru_hole circle (at 3.81 0 90) (size 1.524 1.524) (drill 0.889) (layers *.Cu *.Mask F.SilkS) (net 7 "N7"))
  (pad 8 thru_hole circle (at 6.35 0 90) (size 1.524 1.524) (drill 0.889) (layers *.Cu *.Mask F.SilkS) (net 8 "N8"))
  (pad 9 thru_hole circle (at 8.89 0 90) (size 1.524 1.524) (drill 0.889) (layers *.Cu *.Mask F.SilkS) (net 9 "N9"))
  (pad 10 thru_hole circle (at 11.43 0 90) (size 1.524 1.524) (drill 0.889) (layers *.Cu *.Mask F.SilkS) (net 10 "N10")))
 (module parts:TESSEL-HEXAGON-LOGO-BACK (layer B.Cu) (at 144.145 101.6 270)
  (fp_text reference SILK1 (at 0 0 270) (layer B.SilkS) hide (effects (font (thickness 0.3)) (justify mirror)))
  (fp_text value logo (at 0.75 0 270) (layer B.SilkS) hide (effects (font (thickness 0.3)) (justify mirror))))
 (gr_line (start 127 87.63) (end 161.925 87.63) (layer Edge.Cuts) (width 0.2))
 (gr_line (start 127 87.63) (end 127 115.57) (layer Edge.Cuts) (width 0.2))
 (gr_line (start 127 115.57) (end 161.925 115.57) (layer Edge.Cuts) (width 0.2))
 (gr_line (start 165.1 90.805) (end 165.1 112.395) (layer Edge.Cuts) (width 0.2))
 (gr_arc (start 161.925 90.805) (end 161.925 87.63) (angle 90) (layer Edge.Cuts) (width 0.2))
 (gr_arc (start 161.925 112.395) (end 165.1 112.395) (angle 90) (layer Edge.Cuts) (width 0.2))
 (via (at 1132.715 92.71) (size 1.524) (drill 0.889) (layers F.Cu B.Cu) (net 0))
 (via (at 1132.715 92.71) (size 1.524) (drill 0.889) (layers F.Cu B.Cu) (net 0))
 (via (at 1132.715 92.71) (size 1.524) (drill 0.889) (layers F.Cu B.Cu) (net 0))
 (via (at 1132.715 92.71) (size 1.524) (drill 0.889) (layers F.Cu B.Cu) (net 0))
 (via (at 1132.715 92.71) (size 1.524) (drill 0.889) (layers F.Cu B.Cu) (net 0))
 (via (at 1132.715 92.71) (size 1.524) (drill 0.889) (layers F.Cu B.Cu) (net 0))
 (via (at 1132.715 92.71) (size 1.524) (drill 0.889) (layers F.Cu B.Cu) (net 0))
 (via (at 1132.715 92.71) (size 1.524) (drill 0.889) (layers F.Cu B.Cu) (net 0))
 (via (at 1132.715 92.71) (size 1.524) (drill 0.889) (layers F.Cu B.Cu) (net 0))
 (via (at 1132.715 92.71) (size 1.524) (drill 0.889) (layers F.Cu B.Cu) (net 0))
 (segment (start 132.08 113.03) (end 134.62 113.03) (width 0.635) (layer F.Cu) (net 1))
 (segment (start 132.08 113.03) (end 134.62 113.03) (width 0.635) (layer B.Cu) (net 1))
 (segment (start 134.62 113.03) (end 133.35 113.03) (width 1.143) (layer F.Cu) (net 1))
 (segment (start 133.35 113.03) (end 132.08 113.03) (width 1.143) (layer F.Cu) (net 1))
 (segment (start 132.08 113.03) (end 129.858406 113.03) (width 1.143) (layer F.Cu) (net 1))
 (segment (start 128.905 113.03) (end 129.858406 113.03) (width 1.143) (layer F.Cu) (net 1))
 (segment (start 163.068 114.554) (end 163.576 114.046) (width 0.635) (layer F.Cu) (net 1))
 (segment (start 136.144 114.554) (end 163.068 114.554) (width 0.635) (layer F.Cu) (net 1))
 (segment (start 134.62 113.03) (end 136.144 114.554) (width 0.635) (layer F.Cu) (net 1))
 (segment (start 163.068 114.554) (end 163.576 114.046) (width 0.635) (layer B.Cu) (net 1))
 (segment (start 136.144 114.554) (end 163.068 114.554) (width 0.635) (layer B.Cu) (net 1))
 (segment (start 134.62 113.03) (end 136.144 114.554) (width 0.635) (layer B.Cu) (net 1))
 (segment (start 132.08 110.49) (end 133.35 110.49) (width 1.143) (layer F.Cu) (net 2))
 (segment (start 133.35 110.49) (end 134.62 110.49) (width 1.143) (layer F.Cu) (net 2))
 (segment (start 128.905 110.49) (end 132.08 110.49) (width 1.143) (layer F.Cu) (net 2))
 (segment (start 163.068 88.646) (end 163.576 89.154) (width 0.635) (layer B.Cu) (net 2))
 (segment (start 128.455418 88.646) (end 163.068 88.646) (width 0.635) (layer B.Cu) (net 2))
 (segment (start 127.571499 89.529919) (end 128.455418 88.646) (width 0.635) (layer B.Cu) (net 2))
 (segment (start 127.571499 109.029499) (end 127.571499 89.529919) (width 0.635) (layer B.Cu) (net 2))
 (segment (start 129.032 110.49) (end 127.571499 109.029499) (width 0.635) (layer B.Cu) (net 2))
 (segment (start 132.08 110.49) (end 129.032 110.49) (width 0.635) (layer B.Cu) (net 2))
 (segment (start 163.068 88.646) (end 163.576 89.154) (width 0.635) (layer F.Cu) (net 2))
 (segment (start 127.571499 89.529919) (end 128.455418 88.646) (width 0.635) (layer F.Cu) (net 2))
 (segment (start 128.455418 88.646) (end 163.068 88.646) (width 0.635) (layer F.Cu) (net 2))
 (segment (start 127.571499 109.029499) (end 127.571499 89.529919) (width 0.635) (layer F.Cu) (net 2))
 (segment (start 129.032 110.49) (end 127.571499 109.029499) (width 0.635) (layer F.Cu) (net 2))
 (segment (start 132.08 110.49) (end 129.032 110.49) (width 0.635) (layer F.Cu) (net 2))
 (segment (start 134.62 107.95) (end 133.35 107.95) (width 1.143) (layer F.Cu) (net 3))
 (segment (start 133.35 107.95) (end 132.08 107.95) (width 1.143) (layer F.Cu) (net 3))
 (segment (start 128.905 107.95) (end 132.08 107.95) (width 1.143) (layer F.Cu) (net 3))
 (segment (start 132.08 105.41) (end 133.35 105.41) (width 1.143) (layer F.Cu) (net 4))
 (segment (start 133.35 105.41) (end 134.62 105.41) (width 1.143) (layer F.Cu) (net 4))
 (segment (start 128.905 105.41) (end 132.08 105.41) (width 1.143) (layer F.Cu) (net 4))
 (segment (start 134.62 102.87) (end 133.35 102.87) (width 1.143) (layer F.Cu) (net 5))
 (segment (start 134.62 102.87) (end 132.08 102.87) (width 1.143) (layer F.Cu) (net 5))
 (segment (start 132.08 102.87) (end 128.905 102.87) (width 1.143) (layer F.Cu) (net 5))
 (segment (start 132.08 100.33) (end 133.35 100.33) (width 1.143) (layer F.Cu) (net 6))
 (segment (start 133.35 100.33) (end 134.62 100.33) (width 1.143) (layer F.Cu) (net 6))
 (segment (start 128.905 100.33) (end 132.08 100.33) (width 1.143) (layer F.Cu) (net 6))
 (segment (start 134.62 97.79) (end 133.35 97.79) (width 1.143) (layer F.Cu) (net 7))
 (segment (start 133.35 97.79) (end 132.08 97.79) (width 1.143) (layer F.Cu) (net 7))
 (segment (start 128.905 97.79) (end 132.08 97.79) (width 1.143) (layer F.Cu) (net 7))
 (segment (start 132.08 95.25) (end 133.35 95.25) (width 1.143) (layer F.Cu) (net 8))
 (segment (start 133.35 95.25) (end 134.62 95.25) (width 1.143) (layer F.Cu) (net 8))
 (segment (start 128.905 95.25) (end 132.08 95.25) (width 1.143) (layer F.Cu) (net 8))
 (segment (start 134.62 92.71) (end 133.35 92.71) (width 1.143) (layer F.Cu) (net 9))
 (segment (start 133.35 92.71) (end 132.08 92.71) (width 1.143) (layer F.Cu) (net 9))
 (segment (start 128.905 92.71) (end 132.08 92.71) (width 1.143) (layer F.Cu) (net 9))
 (segment (start 132.08 90.17) (end 133.35 90.17) (width 1.143) (layer F.Cu) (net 10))
 (segment (start 134.62 90.17) (end 133.35 90.17) (width 1.143) (layer F.Cu) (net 10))
 (segment (start 128.905 90.17) (end 132.08 90.17) (width 1.143) (layer F.Cu) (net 10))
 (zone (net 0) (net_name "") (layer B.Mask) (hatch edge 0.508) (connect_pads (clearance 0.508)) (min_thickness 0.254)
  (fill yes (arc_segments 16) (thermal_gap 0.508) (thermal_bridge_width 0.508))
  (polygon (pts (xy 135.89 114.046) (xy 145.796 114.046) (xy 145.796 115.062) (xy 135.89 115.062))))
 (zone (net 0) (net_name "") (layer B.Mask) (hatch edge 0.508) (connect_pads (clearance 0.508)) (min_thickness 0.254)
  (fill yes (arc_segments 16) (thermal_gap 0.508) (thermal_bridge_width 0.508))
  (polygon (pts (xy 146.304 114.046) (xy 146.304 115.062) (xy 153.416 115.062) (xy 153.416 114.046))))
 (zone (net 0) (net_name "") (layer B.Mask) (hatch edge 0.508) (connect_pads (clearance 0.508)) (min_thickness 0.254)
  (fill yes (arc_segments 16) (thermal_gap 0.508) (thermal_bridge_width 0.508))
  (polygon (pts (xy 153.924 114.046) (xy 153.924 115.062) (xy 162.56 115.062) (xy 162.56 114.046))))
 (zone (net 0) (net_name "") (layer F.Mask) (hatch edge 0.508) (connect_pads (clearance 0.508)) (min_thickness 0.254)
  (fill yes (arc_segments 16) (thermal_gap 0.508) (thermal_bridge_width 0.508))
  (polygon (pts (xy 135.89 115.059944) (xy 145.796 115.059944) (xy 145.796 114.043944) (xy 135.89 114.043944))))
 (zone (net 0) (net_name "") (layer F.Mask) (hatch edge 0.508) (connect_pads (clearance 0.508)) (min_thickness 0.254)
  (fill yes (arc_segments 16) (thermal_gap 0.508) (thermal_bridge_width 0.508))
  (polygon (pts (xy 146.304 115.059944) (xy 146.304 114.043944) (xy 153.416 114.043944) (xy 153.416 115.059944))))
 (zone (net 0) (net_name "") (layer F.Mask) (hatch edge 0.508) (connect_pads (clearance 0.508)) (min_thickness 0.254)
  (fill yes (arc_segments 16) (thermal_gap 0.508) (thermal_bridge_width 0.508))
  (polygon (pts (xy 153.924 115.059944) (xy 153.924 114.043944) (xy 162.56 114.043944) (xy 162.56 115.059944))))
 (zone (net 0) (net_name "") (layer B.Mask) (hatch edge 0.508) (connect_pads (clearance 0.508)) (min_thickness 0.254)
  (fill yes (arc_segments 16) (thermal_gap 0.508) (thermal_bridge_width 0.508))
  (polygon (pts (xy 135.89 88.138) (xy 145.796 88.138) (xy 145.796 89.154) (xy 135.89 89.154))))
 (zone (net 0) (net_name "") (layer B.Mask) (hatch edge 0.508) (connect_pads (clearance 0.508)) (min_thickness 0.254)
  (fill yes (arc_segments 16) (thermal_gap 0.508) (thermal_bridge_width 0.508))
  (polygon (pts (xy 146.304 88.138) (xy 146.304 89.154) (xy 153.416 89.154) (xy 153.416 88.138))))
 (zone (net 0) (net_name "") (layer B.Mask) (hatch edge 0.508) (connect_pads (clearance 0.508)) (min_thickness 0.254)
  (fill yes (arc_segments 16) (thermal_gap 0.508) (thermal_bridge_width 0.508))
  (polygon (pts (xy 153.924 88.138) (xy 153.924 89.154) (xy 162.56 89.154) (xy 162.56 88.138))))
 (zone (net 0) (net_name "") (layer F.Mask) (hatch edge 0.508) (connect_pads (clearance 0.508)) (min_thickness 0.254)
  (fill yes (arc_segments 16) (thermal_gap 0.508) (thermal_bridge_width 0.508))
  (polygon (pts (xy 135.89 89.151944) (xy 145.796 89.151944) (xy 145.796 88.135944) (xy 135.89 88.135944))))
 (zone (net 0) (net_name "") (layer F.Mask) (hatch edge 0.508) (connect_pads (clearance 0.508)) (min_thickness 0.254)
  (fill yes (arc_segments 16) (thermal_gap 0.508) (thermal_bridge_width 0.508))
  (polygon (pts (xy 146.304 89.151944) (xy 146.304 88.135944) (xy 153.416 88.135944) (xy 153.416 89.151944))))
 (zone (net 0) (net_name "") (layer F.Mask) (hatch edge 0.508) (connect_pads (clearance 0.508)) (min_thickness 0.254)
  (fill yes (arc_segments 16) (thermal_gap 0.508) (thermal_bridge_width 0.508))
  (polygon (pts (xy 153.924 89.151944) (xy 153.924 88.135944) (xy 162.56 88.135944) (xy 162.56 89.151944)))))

